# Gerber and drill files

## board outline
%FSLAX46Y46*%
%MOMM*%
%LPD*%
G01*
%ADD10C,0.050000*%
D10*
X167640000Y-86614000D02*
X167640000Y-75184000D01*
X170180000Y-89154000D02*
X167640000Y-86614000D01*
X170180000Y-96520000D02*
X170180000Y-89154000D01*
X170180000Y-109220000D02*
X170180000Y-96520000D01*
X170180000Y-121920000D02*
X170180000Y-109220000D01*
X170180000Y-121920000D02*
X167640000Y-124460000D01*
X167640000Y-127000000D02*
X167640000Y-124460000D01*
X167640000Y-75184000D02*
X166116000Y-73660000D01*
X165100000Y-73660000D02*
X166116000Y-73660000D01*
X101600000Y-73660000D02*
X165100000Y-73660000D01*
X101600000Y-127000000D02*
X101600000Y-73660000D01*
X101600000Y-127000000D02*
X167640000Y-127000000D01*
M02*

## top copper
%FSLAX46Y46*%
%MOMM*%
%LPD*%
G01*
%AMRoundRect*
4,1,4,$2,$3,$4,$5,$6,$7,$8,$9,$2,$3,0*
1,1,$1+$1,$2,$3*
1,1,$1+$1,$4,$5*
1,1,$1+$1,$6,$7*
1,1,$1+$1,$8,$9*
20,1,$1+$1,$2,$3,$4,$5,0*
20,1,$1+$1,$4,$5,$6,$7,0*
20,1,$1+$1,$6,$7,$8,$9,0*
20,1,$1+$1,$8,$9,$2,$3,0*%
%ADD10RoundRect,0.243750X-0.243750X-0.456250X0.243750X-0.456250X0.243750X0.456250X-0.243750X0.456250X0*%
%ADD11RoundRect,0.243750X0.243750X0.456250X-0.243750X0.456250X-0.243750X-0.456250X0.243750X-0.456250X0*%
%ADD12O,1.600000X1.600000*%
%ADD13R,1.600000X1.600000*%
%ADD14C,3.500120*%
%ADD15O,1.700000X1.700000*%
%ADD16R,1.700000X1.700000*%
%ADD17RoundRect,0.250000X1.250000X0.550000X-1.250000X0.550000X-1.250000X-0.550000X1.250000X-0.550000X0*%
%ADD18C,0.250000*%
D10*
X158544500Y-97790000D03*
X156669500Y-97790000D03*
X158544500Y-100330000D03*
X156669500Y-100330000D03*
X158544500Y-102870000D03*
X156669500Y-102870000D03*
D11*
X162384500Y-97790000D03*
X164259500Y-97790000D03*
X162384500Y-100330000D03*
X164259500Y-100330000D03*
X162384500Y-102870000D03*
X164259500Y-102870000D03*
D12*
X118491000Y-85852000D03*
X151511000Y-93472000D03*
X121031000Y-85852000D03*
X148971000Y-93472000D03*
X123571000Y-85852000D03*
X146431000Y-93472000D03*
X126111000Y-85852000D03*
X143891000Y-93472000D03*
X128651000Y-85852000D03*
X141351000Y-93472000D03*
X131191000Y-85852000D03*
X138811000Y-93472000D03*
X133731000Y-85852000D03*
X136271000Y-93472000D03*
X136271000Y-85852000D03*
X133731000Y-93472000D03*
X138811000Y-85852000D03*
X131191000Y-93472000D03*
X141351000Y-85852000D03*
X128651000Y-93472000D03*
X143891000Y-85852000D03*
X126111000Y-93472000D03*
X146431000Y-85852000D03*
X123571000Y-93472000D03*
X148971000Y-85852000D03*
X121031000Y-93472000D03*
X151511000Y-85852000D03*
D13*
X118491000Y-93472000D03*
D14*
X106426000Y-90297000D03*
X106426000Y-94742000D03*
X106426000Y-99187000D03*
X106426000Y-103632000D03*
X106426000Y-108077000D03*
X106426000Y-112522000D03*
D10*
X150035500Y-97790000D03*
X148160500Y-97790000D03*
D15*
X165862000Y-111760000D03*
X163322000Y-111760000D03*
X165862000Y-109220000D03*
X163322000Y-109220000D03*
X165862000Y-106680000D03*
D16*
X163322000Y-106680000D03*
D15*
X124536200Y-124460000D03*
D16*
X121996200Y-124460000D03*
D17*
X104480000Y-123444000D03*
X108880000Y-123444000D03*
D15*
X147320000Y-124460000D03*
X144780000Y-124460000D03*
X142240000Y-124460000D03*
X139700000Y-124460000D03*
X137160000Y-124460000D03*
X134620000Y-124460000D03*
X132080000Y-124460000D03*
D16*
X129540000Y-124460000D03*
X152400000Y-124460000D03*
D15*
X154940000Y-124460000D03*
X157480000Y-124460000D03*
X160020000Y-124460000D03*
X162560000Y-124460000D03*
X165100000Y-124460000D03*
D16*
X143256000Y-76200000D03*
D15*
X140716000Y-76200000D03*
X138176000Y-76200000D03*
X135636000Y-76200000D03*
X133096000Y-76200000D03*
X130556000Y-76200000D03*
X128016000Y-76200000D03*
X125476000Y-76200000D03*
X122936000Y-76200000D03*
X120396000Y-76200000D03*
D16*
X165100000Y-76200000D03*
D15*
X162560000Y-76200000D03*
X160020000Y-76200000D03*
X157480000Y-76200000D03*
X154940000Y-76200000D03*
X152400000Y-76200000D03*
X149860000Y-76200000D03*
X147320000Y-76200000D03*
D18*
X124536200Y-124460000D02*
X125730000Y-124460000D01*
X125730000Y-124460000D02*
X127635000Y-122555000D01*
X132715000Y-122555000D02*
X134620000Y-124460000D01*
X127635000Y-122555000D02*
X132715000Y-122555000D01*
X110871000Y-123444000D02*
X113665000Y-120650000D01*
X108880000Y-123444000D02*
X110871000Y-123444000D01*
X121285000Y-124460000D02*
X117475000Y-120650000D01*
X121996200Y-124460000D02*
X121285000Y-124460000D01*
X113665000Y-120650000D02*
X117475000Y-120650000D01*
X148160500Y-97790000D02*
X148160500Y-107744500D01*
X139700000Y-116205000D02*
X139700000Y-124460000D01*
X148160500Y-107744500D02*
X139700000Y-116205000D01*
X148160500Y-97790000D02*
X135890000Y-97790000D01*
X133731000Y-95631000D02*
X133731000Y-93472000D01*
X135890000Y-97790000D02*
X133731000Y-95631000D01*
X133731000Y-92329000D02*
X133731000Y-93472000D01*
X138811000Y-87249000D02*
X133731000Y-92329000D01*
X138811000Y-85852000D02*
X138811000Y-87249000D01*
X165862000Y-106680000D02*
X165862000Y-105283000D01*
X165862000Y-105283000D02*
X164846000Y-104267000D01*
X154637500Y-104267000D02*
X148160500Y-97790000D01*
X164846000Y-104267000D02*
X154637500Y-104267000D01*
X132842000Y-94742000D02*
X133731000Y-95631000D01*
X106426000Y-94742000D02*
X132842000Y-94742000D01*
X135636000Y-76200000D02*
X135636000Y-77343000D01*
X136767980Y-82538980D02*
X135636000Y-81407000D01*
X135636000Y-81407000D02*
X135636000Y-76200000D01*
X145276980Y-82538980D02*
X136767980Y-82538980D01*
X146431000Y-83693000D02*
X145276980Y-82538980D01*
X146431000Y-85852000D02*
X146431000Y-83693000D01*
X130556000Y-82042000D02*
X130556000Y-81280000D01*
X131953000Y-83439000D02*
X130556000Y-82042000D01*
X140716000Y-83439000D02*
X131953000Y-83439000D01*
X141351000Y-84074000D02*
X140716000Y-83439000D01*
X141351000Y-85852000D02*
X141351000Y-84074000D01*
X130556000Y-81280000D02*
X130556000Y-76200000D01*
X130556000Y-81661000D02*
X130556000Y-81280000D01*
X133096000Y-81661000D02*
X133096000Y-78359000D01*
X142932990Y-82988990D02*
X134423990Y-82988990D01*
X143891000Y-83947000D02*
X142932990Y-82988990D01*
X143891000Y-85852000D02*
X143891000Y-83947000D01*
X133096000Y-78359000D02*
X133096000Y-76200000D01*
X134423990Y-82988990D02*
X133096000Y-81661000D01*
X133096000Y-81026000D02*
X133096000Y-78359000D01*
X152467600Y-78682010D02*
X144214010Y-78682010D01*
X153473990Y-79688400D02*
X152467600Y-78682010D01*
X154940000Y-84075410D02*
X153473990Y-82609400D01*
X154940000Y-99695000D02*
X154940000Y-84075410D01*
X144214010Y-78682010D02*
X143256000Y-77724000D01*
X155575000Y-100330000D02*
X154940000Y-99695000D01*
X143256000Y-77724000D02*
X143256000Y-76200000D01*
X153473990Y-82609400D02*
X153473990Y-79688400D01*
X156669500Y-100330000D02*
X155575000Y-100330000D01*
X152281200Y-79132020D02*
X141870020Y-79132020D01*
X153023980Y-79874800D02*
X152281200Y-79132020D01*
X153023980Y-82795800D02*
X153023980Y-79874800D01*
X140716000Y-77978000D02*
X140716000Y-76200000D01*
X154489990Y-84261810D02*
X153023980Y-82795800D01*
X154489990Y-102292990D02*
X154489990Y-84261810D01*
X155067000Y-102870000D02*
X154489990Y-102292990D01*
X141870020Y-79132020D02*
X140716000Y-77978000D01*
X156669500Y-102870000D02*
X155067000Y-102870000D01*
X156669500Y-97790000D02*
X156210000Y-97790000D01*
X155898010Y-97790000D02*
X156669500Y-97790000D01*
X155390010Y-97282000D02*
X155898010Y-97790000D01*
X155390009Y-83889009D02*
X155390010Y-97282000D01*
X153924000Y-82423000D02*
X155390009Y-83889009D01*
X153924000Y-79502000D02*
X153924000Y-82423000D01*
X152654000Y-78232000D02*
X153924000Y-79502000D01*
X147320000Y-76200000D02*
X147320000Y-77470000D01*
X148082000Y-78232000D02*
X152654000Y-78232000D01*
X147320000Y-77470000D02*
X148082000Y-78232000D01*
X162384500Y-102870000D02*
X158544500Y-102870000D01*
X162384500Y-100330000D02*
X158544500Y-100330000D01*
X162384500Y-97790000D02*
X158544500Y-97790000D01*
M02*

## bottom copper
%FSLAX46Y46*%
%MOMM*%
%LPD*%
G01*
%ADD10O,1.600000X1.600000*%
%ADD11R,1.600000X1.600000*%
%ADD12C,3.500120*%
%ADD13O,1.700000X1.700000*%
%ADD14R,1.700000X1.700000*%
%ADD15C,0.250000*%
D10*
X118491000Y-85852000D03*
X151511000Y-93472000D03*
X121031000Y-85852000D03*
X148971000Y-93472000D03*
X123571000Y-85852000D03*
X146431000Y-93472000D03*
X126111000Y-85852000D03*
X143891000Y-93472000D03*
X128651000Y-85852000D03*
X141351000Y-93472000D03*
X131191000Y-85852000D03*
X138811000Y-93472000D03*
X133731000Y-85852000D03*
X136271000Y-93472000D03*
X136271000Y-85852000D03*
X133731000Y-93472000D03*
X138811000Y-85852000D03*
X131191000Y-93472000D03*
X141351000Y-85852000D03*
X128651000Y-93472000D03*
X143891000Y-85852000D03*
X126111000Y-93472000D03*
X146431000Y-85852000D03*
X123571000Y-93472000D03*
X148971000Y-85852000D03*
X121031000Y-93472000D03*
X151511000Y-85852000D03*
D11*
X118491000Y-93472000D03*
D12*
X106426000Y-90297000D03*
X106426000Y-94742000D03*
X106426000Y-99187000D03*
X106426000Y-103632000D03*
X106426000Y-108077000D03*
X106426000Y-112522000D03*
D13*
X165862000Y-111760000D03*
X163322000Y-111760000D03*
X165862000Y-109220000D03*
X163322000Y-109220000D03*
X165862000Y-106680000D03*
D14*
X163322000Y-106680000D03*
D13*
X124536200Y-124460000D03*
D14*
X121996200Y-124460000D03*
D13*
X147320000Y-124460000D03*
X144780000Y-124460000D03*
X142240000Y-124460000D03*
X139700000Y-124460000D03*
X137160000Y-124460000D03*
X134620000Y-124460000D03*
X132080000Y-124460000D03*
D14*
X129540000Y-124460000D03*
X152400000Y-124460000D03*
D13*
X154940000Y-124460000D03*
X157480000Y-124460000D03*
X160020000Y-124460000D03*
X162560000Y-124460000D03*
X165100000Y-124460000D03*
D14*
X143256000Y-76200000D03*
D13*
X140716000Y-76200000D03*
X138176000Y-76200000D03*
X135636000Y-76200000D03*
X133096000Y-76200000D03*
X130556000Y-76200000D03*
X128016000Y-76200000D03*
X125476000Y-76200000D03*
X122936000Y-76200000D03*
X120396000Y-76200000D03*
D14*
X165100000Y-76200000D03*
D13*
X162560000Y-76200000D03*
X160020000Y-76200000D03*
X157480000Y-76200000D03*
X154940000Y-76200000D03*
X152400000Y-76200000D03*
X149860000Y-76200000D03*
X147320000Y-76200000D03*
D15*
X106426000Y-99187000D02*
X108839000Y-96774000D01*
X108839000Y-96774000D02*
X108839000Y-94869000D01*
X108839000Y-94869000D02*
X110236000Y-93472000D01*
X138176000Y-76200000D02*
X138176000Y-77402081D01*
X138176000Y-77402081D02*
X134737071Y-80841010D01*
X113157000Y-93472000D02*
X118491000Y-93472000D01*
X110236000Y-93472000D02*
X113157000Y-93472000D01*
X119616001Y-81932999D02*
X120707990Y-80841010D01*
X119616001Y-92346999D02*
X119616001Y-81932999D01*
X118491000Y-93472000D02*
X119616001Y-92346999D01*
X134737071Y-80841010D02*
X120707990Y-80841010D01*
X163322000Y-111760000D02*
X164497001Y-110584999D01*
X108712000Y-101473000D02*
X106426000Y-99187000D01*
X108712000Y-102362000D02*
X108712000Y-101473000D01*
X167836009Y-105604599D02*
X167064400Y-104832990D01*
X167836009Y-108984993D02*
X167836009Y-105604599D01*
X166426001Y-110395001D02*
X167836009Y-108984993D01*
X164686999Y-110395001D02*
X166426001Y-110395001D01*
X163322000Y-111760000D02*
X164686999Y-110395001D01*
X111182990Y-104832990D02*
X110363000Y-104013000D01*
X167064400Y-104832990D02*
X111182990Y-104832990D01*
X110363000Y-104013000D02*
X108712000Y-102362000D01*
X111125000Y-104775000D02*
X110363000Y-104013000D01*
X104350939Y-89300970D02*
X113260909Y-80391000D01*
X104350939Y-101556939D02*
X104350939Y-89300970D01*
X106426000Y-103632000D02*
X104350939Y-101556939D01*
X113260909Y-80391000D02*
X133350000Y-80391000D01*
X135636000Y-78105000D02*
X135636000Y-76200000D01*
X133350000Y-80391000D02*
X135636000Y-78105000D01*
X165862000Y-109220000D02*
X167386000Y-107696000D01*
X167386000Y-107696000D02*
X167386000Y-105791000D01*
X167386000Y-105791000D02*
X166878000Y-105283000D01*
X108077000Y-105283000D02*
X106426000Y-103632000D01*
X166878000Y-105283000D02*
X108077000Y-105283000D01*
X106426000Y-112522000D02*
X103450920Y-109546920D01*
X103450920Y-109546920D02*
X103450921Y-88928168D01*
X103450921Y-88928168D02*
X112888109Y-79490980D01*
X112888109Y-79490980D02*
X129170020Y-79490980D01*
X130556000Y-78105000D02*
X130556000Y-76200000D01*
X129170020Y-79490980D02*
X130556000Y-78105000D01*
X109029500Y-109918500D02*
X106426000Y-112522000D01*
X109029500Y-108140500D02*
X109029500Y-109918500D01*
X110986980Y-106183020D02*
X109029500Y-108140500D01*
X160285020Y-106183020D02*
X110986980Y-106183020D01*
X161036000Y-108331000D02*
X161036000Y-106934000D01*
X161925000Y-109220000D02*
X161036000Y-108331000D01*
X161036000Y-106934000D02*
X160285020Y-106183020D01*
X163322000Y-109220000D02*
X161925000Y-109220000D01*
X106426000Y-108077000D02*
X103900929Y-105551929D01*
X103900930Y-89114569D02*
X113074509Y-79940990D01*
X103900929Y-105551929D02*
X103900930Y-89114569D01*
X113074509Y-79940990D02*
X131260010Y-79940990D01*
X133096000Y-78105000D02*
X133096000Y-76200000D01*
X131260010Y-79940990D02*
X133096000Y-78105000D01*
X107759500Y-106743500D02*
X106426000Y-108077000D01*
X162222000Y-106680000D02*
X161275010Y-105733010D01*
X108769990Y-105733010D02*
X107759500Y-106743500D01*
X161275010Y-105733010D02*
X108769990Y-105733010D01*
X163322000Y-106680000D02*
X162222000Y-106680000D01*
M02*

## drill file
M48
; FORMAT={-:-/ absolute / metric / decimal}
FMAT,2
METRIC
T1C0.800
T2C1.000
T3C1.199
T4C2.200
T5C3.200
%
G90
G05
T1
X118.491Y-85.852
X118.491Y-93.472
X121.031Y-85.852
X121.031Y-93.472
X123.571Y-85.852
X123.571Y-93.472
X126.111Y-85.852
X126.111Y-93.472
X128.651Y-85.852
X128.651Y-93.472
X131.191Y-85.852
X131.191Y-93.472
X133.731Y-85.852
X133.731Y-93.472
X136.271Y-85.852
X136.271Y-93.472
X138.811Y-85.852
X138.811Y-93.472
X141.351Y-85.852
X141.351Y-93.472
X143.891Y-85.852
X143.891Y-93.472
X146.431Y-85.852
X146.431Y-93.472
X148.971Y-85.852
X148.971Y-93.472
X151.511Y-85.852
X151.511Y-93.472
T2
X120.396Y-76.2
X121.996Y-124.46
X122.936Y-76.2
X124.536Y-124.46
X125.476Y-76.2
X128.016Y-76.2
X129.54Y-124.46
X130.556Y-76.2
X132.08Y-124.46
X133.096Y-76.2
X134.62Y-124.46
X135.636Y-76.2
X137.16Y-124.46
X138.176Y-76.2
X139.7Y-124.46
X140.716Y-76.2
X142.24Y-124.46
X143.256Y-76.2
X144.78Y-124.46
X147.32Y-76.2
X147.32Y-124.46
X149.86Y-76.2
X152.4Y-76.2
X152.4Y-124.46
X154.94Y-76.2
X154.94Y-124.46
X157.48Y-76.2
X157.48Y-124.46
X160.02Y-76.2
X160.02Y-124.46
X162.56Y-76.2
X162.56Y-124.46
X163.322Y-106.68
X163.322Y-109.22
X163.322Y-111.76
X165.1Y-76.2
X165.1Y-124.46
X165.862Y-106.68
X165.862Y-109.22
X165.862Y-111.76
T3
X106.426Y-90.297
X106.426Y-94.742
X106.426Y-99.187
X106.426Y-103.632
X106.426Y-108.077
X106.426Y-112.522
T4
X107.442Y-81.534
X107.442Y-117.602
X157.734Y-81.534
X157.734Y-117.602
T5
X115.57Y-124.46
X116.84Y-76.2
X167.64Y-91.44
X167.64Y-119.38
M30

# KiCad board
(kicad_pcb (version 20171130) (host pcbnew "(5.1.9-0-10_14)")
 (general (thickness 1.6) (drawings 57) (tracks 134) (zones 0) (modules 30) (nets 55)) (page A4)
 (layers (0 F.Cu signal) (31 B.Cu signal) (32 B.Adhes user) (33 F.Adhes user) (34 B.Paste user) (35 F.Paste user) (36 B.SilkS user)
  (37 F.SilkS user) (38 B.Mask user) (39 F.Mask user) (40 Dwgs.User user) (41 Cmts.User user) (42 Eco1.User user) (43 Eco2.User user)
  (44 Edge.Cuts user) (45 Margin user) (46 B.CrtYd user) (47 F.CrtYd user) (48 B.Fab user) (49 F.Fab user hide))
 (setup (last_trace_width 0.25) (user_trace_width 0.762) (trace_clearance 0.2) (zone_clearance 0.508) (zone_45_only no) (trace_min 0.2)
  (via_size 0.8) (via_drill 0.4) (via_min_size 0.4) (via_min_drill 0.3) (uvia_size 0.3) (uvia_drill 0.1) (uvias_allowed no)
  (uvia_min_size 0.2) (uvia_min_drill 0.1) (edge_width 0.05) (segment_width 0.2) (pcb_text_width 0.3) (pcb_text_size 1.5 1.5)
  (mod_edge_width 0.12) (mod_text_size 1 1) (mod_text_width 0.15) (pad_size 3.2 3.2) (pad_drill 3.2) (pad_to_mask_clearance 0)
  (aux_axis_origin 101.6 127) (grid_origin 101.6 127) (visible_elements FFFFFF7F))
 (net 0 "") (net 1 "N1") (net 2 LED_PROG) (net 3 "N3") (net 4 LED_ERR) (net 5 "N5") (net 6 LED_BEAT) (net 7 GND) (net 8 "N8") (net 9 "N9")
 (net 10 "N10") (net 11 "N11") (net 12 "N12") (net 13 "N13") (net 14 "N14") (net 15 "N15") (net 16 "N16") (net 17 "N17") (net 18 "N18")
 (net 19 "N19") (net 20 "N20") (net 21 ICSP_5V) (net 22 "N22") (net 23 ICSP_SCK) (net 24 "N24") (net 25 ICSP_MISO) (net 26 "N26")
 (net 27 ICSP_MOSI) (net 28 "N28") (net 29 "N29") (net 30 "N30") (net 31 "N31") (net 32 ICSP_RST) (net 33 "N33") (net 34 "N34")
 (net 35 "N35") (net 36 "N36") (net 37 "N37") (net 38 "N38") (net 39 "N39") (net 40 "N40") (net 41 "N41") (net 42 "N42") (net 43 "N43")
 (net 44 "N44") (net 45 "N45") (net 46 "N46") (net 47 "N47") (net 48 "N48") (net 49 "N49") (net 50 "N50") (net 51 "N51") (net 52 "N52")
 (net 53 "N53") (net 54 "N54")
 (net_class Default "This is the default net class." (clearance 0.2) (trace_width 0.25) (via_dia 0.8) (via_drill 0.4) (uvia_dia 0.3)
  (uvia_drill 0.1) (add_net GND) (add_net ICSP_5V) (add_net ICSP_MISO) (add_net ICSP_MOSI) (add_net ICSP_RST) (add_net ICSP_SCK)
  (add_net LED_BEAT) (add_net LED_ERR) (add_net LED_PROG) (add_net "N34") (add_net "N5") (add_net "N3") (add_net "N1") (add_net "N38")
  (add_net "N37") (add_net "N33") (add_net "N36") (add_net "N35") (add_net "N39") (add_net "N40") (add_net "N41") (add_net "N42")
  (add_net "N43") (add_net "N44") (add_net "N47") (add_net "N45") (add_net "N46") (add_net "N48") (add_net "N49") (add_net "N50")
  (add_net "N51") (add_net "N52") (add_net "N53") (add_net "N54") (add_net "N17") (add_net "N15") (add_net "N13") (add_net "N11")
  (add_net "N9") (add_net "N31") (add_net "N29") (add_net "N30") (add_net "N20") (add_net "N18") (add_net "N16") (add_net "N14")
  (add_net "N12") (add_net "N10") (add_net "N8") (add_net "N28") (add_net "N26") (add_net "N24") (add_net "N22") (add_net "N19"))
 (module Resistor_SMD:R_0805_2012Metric (layer F.Cu) (at 157.607 97.79)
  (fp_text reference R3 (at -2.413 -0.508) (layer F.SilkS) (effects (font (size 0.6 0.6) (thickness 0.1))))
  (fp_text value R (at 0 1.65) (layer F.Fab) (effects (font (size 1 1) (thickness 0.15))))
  (pad 2 smd roundrect (at 0.9375 0) (size 0.975 1.4) (layers F.Cu F.Paste F.Mask) (roundrect_rratio 0.25) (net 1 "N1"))
  (pad 1 smd roundrect (at -0.9375 0) (size 0.975 1.4) (layers F.Cu F.Paste F.Mask) (roundrect_rratio 0.25) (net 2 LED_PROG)))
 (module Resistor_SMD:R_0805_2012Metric (layer F.Cu) (at 157.607 100.33)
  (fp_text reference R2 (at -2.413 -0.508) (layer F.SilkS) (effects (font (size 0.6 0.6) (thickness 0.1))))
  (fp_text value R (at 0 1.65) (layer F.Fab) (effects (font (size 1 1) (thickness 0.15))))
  (pad 2 smd roundrect (at 0.9375 0) (size 0.975 1.4) (layers F.Cu F.Paste F.Mask) (roundrect_rratio 0.25) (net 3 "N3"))
  (pad 1 smd roundrect (at -0.9375 0) (size 0.975 1.4) (layers F.Cu F.Paste F.Mask) (roundrect_rratio 0.25) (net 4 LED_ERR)))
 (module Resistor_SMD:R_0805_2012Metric (layer F.Cu) (at 157.607 102.87)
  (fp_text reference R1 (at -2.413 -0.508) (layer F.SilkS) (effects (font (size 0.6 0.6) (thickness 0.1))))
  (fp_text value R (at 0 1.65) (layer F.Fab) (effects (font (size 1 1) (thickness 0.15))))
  (pad 2 smd roundrect (at 0.9375 0) (size 0.975 1.4) (layers F.Cu F.Paste F.Mask) (roundrect_rratio 0.25) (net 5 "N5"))
  (pad 1 smd roundrect (at -0.9375 0) (size 0.975 1.4) (layers F.Cu F.Paste F.Mask) (roundrect_rratio 0.25) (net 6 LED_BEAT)))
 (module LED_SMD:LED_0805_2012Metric (layer F.Cu) (at 163.322 97.79 180)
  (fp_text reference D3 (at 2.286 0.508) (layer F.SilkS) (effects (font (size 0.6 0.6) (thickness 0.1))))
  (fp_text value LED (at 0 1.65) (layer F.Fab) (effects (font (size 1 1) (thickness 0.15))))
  (pad 2 smd roundrect (at 0.9375 0 180) (size 0.975 1.4) (layers F.Cu F.Paste F.Mask) (roundrect_rratio 0.25) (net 1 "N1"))
  (pad 1 smd roundrect (at -0.9375 0 180) (size 0.975 1.4) (layers F.Cu F.Paste F.Mask) (roundrect_rratio 0.25) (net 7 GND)))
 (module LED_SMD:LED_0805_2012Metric (layer F.Cu) (at 163.322 100.33 180)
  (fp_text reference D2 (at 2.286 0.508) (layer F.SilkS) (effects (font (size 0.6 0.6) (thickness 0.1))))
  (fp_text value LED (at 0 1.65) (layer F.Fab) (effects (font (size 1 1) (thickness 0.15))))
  (pad 2 smd roundrect (at 0.9375 0 180) (size 0.975 1.4) (layers F.Cu F.Paste F.Mask) (roundrect_rratio 0.25) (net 3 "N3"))
  (pad 1 smd roundrect (at -0.9375 0 180) (size 0.975 1.4) (layers F.Cu F.Paste F.Mask) (roundrect_rratio 0.25) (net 7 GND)))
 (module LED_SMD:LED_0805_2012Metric (layer F.Cu) (at 163.322 102.87 180)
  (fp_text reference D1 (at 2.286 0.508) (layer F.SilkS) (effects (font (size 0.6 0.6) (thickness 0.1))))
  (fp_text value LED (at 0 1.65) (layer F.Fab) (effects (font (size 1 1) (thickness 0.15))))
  (pad 2 smd roundrect (at 0.9375 0 180) (size 0.975 1.4) (layers F.Cu F.Paste F.Mask) (roundrect_rratio 0.25) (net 5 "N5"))
  (pad 1 smd roundrect (at -0.9375 0 180) (size 0.975 1.4) (layers F.Cu F.Paste F.Mask) (roundrect_rratio 0.25) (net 7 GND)))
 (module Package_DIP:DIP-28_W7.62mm (layer F.Cu) (at 118.491 93.472 90)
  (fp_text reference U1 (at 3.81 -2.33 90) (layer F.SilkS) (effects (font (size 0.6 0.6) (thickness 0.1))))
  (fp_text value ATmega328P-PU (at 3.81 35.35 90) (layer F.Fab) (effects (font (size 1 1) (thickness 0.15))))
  (pad 28 thru_hole oval (at 7.62 0 90) (size 1.6 1.6) (drill 0.8) (layers *.Cu *.Mask) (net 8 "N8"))
  (pad 14 thru_hole oval (at 0 33.02 90) (size 1.6 1.6) (drill 0.8) (layers *.Cu *.Mask) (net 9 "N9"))
  (pad 27 thru_hole oval (at 7.62 2.54 90) (size 1.6 1.6) (drill 0.8) (layers *.Cu *.Mask) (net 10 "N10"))
  (pad 13 thru_hole oval (at 0 30.48 90) (size 1.6 1.6) (drill 0.8) (layers *.Cu *.Mask) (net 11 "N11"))
  (pad 26 thru_hole oval (at 7.62 5.08 90) (size 1.6 1.6) (drill 0.8) (layers *.Cu *.Mask) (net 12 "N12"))
  (pad 12 thru_hole oval (at 0 27.94 90) (size 1.6 1.6) (drill 0.8) (layers *.Cu *.Mask) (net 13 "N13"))
  (pad 25 thru_hole oval (at 7.62 7.62 90) (size 1.6 1.6) (drill 0.8) (layers *.Cu *.Mask) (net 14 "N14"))
  (pad 11 thru_hole oval (at 0 25.4 90) (size 1.6 1.6) (drill 0.8) (layers *.Cu *.Mask) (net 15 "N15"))
  (pad 24 thru_hole oval (at 7.62 10.16 90) (size 1.6 1.6) (drill 0.8) (layers *.Cu *.Mask) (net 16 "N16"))
  (pad 10 thru_hole oval (at 0 22.86 90) (size 1.6 1.6) (drill 0.8) (layers *.Cu *.Mask) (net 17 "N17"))
  (pad 23 thru_hole oval (at 7.62 12.7 90) (size 1.6 1.6) (drill 0.8) (layers *.Cu *.Mask) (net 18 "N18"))
  (pad 9 thru_hole oval (at 0 20.32 90) (size 1.6 1.6) (drill 0.8) (layers *.Cu *.Mask) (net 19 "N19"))
  (pad 22 thru_hole oval (at 7.62 15.24 90) (size 1.6 1.6) (drill 0.8) (layers *.Cu *.Mask) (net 7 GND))
  (pad 8 thru_hole oval (at 0 17.78 90) (size 1.6 1.6) (drill 0.8) (layers *.Cu *.Mask) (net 7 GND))
  (pad 21 thru_hole oval (at 7.62 17.78 90) (size 1.6 1.6) (drill 0.8) (layers *.Cu *.Mask) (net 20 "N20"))
  (pad 7 thru_hole oval (at 0 15.24 90) (size 1.6 1.6) (drill 0.8) (layers *.Cu *.Mask) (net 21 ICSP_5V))
  (pad 20 thru_hole oval (at 7.62 20.32 90) (size 1.6 1.6) (drill 0.8) (layers *.Cu *.Mask) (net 21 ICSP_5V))
  (pad 6 thru_hole oval (at 0 12.7 90) (size 1.6 1.6) (drill 0.8) (layers *.Cu *.Mask) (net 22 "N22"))
  (pad 19 thru_hole oval (at 7.62 22.86 90) (size 1.6 1.6) (drill 0.8) (layers *.Cu *.Mask) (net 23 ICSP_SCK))
  (pad 5 thru_hole oval (at 0 10.16 90) (size 1.6 1.6) (drill 0.8) (layers *.Cu *.Mask) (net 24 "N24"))
  (pad 18 thru_hole oval (at 7.62 25.4 90) (size 1.6 1.6) (drill 0.8) (layers *.Cu *.Mask) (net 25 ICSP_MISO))
  (pad 4 thru_hole oval (at 0 7.62 90) (size 1.6 1.6) (drill 0.8) (layers *.Cu *.Mask) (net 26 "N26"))
  (pad 17 thru_hole oval (at 7.62 27.94 90) (size 1.6 1.6) (drill 0.8) (layers *.Cu *.Mask) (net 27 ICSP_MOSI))
  (pad 3 thru_hole oval (at 0 5.08 90) (size 1.6 1.6) (drill 0.8) (layers *.Cu *.Mask) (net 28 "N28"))
  (pad 16 thru_hole oval (at 7.62 30.48 90) (size 1.6 1.6) (drill 0.8) (layers *.Cu *.Mask) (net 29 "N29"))
  (pad 2 thru_hole oval (at 0 2.54 90) (size 1.6 1.6) (drill 0.8) (layers *.Cu *.Mask) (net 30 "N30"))
  (pad 15 thru_hole oval (at 7.62 33.02 90) (size 1.6 1.6) (drill 0.8) (layers *.Cu *.Mask) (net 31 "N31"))
  (pad 1 thru_hole rect (at 0 0 90) (size 1.6 1.6) (drill 0.8) (layers *.Cu *.Mask) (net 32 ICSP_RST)))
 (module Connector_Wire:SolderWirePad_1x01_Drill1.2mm (layer F.Cu) (at 106.426 90.297 90)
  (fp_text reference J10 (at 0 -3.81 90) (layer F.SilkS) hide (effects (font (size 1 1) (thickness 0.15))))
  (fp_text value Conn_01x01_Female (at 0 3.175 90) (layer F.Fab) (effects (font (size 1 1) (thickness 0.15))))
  (pad 1 thru_hole circle (at 0 0 90) (size 3.50012 3.50012) (drill 1.19888) (layers *.Cu *.Mask) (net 7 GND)))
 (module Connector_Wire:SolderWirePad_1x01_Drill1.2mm (layer F.Cu) (at 106.426 94.742 90)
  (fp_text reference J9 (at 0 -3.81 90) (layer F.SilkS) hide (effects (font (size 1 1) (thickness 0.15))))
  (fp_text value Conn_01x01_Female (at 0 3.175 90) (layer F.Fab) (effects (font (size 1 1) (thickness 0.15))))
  (pad 1 thru_hole circle (at 0 0 90) (size 3.50012 3.50012) (drill 1.19888) (layers *.Cu *.Mask) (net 21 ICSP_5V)))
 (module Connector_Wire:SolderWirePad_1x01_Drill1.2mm (layer F.Cu) (at 106.426 99.187 90)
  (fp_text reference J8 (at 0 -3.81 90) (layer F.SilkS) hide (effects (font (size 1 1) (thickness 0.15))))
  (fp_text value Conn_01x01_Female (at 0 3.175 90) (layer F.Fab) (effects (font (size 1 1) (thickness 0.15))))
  (pad 1 thru_hole circle (at 0 0 90) (size 3.50012 3.50012) (drill 1.19888) (layers *.Cu *.Mask) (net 32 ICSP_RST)))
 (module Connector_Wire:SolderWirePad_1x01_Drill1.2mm (layer F.Cu) (at 106.426 103.632 90)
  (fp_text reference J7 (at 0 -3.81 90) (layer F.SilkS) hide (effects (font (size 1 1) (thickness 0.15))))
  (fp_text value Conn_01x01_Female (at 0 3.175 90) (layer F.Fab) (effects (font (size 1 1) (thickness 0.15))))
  (pad 1 thru_hole circle (at 0 0 90) (size 3.50012 3.50012) (drill 1.19888) (layers *.Cu *.Mask) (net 27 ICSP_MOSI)))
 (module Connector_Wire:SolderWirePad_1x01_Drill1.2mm (layer F.Cu) (at 106.426 108.077 90)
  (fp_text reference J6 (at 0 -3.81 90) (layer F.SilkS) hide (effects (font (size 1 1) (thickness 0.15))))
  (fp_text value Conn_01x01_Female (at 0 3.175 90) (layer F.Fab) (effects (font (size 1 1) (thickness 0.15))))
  (pad 1 thru_hole circle (at 0 0 90) (size 3.50012 3.50012) (drill 1.19888) (layers *.Cu *.Mask) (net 25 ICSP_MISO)))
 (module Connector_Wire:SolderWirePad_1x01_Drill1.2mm (layer F.Cu) (at 106.426 112.522 90)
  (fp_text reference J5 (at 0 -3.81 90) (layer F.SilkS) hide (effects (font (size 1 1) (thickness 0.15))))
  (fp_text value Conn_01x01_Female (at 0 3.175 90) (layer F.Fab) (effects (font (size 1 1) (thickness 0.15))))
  (pad 1 thru_hole circle (at 0 0 90) (size 3.50012 3.50012) (drill 1.19888) (layers *.Cu *.Mask) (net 23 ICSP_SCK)))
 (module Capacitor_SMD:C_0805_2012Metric (layer F.Cu) (at 149.098 97.79)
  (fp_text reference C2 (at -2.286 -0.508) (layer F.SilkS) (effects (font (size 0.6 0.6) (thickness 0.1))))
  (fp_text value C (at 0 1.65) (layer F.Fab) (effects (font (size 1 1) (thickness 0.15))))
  (pad 2 smd roundrect (at 0.9375 0) (size 0.975 1.4) (layers F.Cu F.Paste F.Mask) (roundrect_rratio 0.25) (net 7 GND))
  (pad 1 smd roundrect (at -0.9375 0) (size 0.975 1.4) (layers F.Cu F.Paste F.Mask) (roundrect_rratio 0.25) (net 21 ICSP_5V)))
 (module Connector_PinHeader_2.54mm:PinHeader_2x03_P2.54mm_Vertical (layer F.Cu) (at 163.322 106.68)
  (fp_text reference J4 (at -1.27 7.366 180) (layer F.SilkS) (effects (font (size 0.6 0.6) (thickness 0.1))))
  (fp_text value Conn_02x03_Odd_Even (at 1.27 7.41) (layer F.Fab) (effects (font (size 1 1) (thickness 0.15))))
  (pad 6 thru_hole oval (at 2.54 5.08) (size 1.7 1.7) (drill 1) (layers *.Cu *.Mask) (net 7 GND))
  (pad 5 thru_hole oval (at 0 5.08) (size 1.7 1.7) (drill 1) (layers *.Cu *.Mask) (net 32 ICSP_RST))
  (pad 4 thru_hole oval (at 2.54 2.54) (size 1.7 1.7) (drill 1) (layers *.Cu *.Mask) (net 27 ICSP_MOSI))
  (pad 3 thru_hole oval (at 0 2.54) (size 1.7 1.7) (drill 1) (layers *.Cu *.Mask) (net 23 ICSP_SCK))
  (pad 2 thru_hole oval (at 2.54 0) (size 1.7 1.7) (drill 1) (layers *.Cu *.Mask) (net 21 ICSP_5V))
  (pad 1 thru_hole rect (at 0 0) (size 1.7 1.7) (drill 1) (layers *.Cu *.Mask) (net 25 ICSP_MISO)))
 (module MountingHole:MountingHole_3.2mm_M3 (layer F.Cu) (at 115.57 124.46)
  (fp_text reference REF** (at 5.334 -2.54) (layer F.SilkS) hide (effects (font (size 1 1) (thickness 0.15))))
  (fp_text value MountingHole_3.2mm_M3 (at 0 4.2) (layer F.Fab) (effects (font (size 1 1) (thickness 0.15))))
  (pad 1 np_thru_hole circle (at 0 0) (size 3.2 3.2) (drill 3.2) (layers *.Cu *.Mask)))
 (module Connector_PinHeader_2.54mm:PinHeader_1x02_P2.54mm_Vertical (layer F.Cu) (at 121.9962 124.46 90)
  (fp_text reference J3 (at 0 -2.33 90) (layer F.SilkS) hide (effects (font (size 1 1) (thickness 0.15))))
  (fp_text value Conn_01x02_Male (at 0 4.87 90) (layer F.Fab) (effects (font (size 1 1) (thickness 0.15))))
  (pad 2 thru_hole oval (at 0 2.54 90) (size 1.7 1.7) (drill 1) (layers *.Cu *.Mask) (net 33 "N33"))
  (pad 1 thru_hole rect (at 0 0 90) (size 1.7 1.7) (drill 1) (layers *.Cu *.Mask) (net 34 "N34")))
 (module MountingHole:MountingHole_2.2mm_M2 (layer F.Cu) (at 107.442 117.602)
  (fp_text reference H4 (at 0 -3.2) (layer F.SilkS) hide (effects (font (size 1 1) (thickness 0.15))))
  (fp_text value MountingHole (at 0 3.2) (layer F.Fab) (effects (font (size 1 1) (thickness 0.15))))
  (pad 1 np_thru_hole circle (at 0 0) (size 2.2 2.2) (drill 2.2) (layers *.Cu *.Mask)))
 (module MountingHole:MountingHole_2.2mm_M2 (layer F.Cu) (at 107.442 81.534)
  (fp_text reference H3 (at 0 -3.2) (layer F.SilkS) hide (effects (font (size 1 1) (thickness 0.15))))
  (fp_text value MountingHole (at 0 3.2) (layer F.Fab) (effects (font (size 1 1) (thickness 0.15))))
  (pad 1 np_thru_hole circle (at 0 0) (size 2.2 2.2) (drill 2.2) (layers *.Cu *.Mask)))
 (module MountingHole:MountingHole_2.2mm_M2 (layer F.Cu) (at 157.734 81.534)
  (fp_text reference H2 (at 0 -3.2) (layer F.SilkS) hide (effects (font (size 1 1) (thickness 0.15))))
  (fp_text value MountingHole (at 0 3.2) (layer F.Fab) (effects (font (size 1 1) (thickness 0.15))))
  (pad 1 np_thru_hole circle (at 0 0) (size 2.2 2.2) (drill 2.2) (layers *.Cu *.Mask)))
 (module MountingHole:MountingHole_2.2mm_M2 (layer F.Cu) (at 157.734 117.602)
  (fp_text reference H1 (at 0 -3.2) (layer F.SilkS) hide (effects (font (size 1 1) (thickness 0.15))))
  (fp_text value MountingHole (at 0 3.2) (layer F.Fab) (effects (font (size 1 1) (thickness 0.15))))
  (pad 1 np_thru_hole circle (at 0 0) (size 2.2 2.2) (drill 2.2) (layers *.Cu *.Mask)))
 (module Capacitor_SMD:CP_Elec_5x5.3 (layer F.Cu) (at 106.68 123.444 180)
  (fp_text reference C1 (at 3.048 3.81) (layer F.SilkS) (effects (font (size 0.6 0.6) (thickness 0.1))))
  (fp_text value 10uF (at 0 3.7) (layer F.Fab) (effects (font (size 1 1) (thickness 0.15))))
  (pad 2 smd roundrect (at 2.2 0 180) (size 3 1.6) (layers F.Cu F.Paste F.Mask) (roundrect_rratio 0.15625) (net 7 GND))
  (pad 1 smd roundrect (at -2.2 0 180) (size 3 1.6) (layers F.Cu F.Paste F.Mask) (roundrect_rratio 0.15625) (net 34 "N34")))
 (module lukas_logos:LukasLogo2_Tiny (layer F.Cu) (at 157.988 109.22 90)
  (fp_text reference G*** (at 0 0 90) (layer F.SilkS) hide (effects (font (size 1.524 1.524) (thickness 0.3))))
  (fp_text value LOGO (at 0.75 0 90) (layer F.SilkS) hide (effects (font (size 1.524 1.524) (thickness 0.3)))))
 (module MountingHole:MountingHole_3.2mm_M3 (layer F.Cu) (at 116.84 76.2)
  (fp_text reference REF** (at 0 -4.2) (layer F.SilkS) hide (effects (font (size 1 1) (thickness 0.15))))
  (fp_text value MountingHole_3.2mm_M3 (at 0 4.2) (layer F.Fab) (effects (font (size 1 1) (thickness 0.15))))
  (pad 1 np_thru_hole circle (at 0 0) (size 3.2 3.2) (drill 3.2) (layers *.Cu *.Mask)))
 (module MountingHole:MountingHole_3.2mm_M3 (layer F.Cu) (at 167.64 91.44)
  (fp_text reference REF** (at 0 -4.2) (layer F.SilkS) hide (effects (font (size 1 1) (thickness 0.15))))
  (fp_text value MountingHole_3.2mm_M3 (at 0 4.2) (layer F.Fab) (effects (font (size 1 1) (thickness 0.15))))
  (pad 1 np_thru_hole circle (at 0 0) (size 3.2 3.2) (drill 3.2) (layers *.Cu *.Mask)))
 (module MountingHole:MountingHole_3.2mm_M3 (layer F.Cu) (at 167.64 119.38)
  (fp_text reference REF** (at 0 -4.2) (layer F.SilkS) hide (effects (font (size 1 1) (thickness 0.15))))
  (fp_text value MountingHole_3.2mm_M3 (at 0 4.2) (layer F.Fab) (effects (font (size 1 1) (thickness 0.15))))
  (pad 1 np_thru_hole circle (at 0 0) (size 3.2 3.2) (drill 3.2) (layers *.Cu *.Mask)))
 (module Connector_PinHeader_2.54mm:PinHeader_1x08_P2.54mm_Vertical (layer F.Cu) (at 129.54 124.46 90)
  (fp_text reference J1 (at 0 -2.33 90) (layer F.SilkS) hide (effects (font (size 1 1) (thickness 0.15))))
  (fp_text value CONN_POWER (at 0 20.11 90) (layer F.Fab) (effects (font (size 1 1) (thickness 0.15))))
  (pad 8 thru_hole oval (at 0 17.78 90) (size 1.7 1.7) (drill 1) (layers *.Cu *.Mask) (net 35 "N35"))
  (pad 7 thru_hole oval (at 0 15.24 90) (size 1.7 1.7) (drill 1) (layers *.Cu *.Mask) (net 7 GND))
  (pad 6 thru_hole oval (at 0 12.7 90) (size 1.7 1.7) (drill 1) (layers *.Cu *.Mask) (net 7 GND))
  (pad 5 thru_hole oval (at 0 10.16 90) (size 1.7 1.7) (drill 1) (layers *.Cu *.Mask) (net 21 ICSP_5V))
  (pad 4 thru_hole oval (at 0 7.62 90) (size 1.7 1.7) (drill 1) (layers *.Cu *.Mask) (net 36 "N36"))
  (pad 3 thru_hole oval (at 0 5.08 90) (size 1.7 1.7) (drill 1) (layers *.Cu *.Mask) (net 33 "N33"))
  (pad 2 thru_hole oval (at 0 2.54 90) (size 1.7 1.7) (drill 1) (layers *.Cu *.Mask) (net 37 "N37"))
  (pad 1 thru_hole rect (at 0 0 90) (size 1.7 1.7) (drill 1) (layers *.Cu *.Mask) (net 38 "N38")))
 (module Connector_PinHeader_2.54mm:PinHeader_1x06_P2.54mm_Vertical (layer F.Cu) (at 152.4 124.46 90)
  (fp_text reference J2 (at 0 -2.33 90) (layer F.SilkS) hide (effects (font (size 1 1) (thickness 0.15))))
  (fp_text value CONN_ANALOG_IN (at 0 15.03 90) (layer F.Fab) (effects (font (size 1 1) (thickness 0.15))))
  (pad 1 thru_hole rect (at 0 0 90) (size 1.7 1.7) (drill 1) (layers *.Cu *.Mask) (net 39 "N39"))
  (pad 2 thru_hole oval (at 0 2.54 90) (size 1.7 1.7) (drill 1) (layers *.Cu *.Mask) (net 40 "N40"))
  (pad 3 thru_hole oval (at 0 5.08 90) (size 1.7 1.7) (drill 1) (layers *.Cu *.Mask) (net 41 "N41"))
  (pad 4 thru_hole oval (at 0 7.62 90) (size 1.7 1.7) (drill 1) (layers *.Cu *.Mask) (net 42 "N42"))
  (pad 5 thru_hole oval (at 0 10.16 90) (size 1.7 1.7) (drill 1) (layers *.Cu *.Mask) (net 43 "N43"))
  (pad 6 thru_hole oval (at 0 12.7 90) (size 1.7 1.7) (drill 1) (layers *.Cu *.Mask) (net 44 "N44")))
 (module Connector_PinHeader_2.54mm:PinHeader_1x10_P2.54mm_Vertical (layer F.Cu) (at 143.256 76.2 270)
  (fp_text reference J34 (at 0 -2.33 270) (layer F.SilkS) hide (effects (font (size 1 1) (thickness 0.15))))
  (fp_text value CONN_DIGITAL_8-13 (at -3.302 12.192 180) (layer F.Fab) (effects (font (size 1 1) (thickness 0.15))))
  (pad 1 thru_hole rect (at 0 0 270) (size 1.7 1.7) (drill 1) (layers *.Cu *.Mask) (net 4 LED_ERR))
  (pad 2 thru_hole oval (at 0 2.54 270) (size 1.7 1.7) (drill 1) (layers *.Cu *.Mask) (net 6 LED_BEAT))
  (pad 3 thru_hole oval (at 0 5.08 270) (size 1.7 1.7) (drill 1) (layers *.Cu *.Mask) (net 32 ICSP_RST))
  (pad 4 thru_hole oval (at 0 7.62 270) (size 1.7 1.7) (drill 1) (layers *.Cu *.Mask) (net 27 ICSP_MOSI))
  (pad 5 thru_hole oval (at 0 10.16 270) (size 1.7 1.7) (drill 1) (layers *.Cu *.Mask) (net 25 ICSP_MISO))
  (pad 6 thru_hole oval (at 0 12.7 270) (size 1.7 1.7) (drill 1) (layers *.Cu *.Mask) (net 23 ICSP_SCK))
  (pad 7 thru_hole oval (at 0 15.24 270) (size 1.7 1.7) (drill 1) (layers *.Cu *.Mask) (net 7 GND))
  (pad 8 thru_hole oval (at 0 17.78 270) (size 1.7 1.7) (drill 1) (layers *.Cu *.Mask) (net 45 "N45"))
  (pad 9 thru_hole oval (at 0 20.32 270) (size 1.7 1.7) (drill 1) (layers *.Cu *.Mask) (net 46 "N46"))
  (pad 10 thru_hole oval (at 0 22.86 270) (size 1.7 1.7) (drill 1) (layers *.Cu *.Mask) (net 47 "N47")))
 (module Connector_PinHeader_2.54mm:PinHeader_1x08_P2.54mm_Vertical (layer F.Cu) (at 165.1 76.2 270)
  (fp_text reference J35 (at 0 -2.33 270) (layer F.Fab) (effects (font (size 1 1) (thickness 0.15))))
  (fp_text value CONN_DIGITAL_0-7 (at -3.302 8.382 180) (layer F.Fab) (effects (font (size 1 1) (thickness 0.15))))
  (pad 1 thru_hole rect (at 0 0 270) (size 1.7 1.7) (drill 1) (layers *.Cu *.Mask) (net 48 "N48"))
  (pad 2 thru_hole oval (at 0 2.54 270) (size 1.7 1.7) (drill 1) (layers *.Cu *.Mask) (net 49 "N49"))
  (pad 3 thru_hole oval (at 0 5.08 270) (size 1.7 1.7) (drill 1) (layers *.Cu *.Mask) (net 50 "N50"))
  (pad 4 thru_hole oval (at 0 7.62 270) (size 1.7 1.7) (drill 1) (layers *.Cu *.Mask) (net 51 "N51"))
  (pad 5 thru_hole oval (at 0 10.16 270) (size 1.7 1.7) (drill 1) (layers *.Cu *.Mask) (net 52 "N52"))
  (pad 6 thru_hole oval (at 0 12.7 270) (size 1.7 1.7) (drill 1) (layers *.Cu *.Mask) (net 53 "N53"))
  (pad 7 thru_hole oval (at 0 15.24 270) (size 1.7 1.7) (drill 1) (layers *.Cu *.Mask) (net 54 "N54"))
  (pad 8 thru_hole oval (at 0 17.78 270) (size 1.7 1.7) (drill 1) (layers *.Cu *.Mask) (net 2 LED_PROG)))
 (gr_line (start 167.64 86.614) (end 167.64 75.184) (layer Edge.Cuts) (width 0.05))
 (gr_line (start 170.18 89.154) (end 167.64 86.614) (layer Edge.Cuts) (width 0.05))
 (gr_line (start 170.18 96.52) (end 170.18 89.154) (layer Edge.Cuts) (width 0.05))
 (gr_line (start 170.18 109.22) (end 170.18 96.52) (layer Edge.Cuts) (width 0.05))
 (gr_line (start 170.18 121.92) (end 170.18 109.22) (layer Edge.Cuts) (width 0.05))
 (gr_line (start 170.18 121.92) (end 167.64 124.46) (layer Edge.Cuts) (width 0.05))
 (gr_line (start 167.64 127) (end 167.64 124.46) (layer Edge.Cuts) (width 0.05))
 (gr_line (start 167.64 75.184) (end 166.116 73.66) (layer Edge.Cuts) (width 0.05))
 (gr_line (start 165.1 73.66) (end 166.116 73.66) (layer Edge.Cuts) (width 0.05))
 (gr_line (start 101.6 73.66) (end 165.1 73.66) (layer Edge.Cuts) (width 0.05))
 (gr_line (start 101.6 127) (end 101.6 73.66) (layer Edge.Cuts) (width 0.05))
 (gr_line (start 101.6 127) (end 167.64 127) (layer Edge.Cuts) (width 0.05))
 (segment (start 124.5362 124.46) (end 125.73 124.46) (width 0.25) (layer F.Cu) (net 33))
 (segment (start 125.73 124.46) (end 127.635 122.555) (width 0.25) (layer F.Cu) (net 33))
 (segment (start 132.715 122.555) (end 134.62 124.46) (width 0.25) (layer F.Cu) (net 33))
 (segment (start 127.635 122.555) (end 132.715 122.555) (width 0.25) (layer F.Cu) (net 33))
 (segment (start 110.871 123.444) (end 113.665 120.65) (width 0.25) (layer F.Cu) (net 34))
 (segment (start 108.88 123.444) (end 110.871 123.444) (width 0.25) (layer F.Cu) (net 34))
 (segment (start 121.285 124.46) (end 117.475 120.65) (width 0.25) (layer F.Cu) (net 34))
 (segment (start 121.9962 124.46) (end 121.285 124.46) (width 0.25) (layer F.Cu) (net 34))
 (segment (start 113.665 120.65) (end 117.475 120.65) (width 0.25) (layer F.Cu) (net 34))
 (segment (start 148.1605 97.79) (end 148.1605 107.7445) (width 0.25) (layer F.Cu) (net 21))
 (segment (start 139.7 116.205) (end 139.7 124.46) (width 0.25) (layer F.Cu) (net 21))
 (segment (start 148.1605 107.7445) (end 139.7 116.205) (width 0.25) (layer F.Cu) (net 21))
 (segment (start 148.1605 97.79) (end 135.89 97.79) (width 0.25) (layer F.Cu) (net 21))
 (segment (start 133.731 95.631) (end 133.731 93.472) (width 0.25) (layer F.Cu) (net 21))
 (segment (start 135.89 97.79) (end 133.731 95.631) (width 0.25) (layer F.Cu) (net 21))
 (segment (start 133.731 92.329) (end 133.731 93.472) (width 0.25) (layer F.Cu) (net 21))
 (segment (start 138.811 87.249) (end 133.731 92.329) (width 0.25) (layer F.Cu) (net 21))
 (segment (start 138.811 85.852) (end 138.811 87.249) (width 0.25) (layer F.Cu) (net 21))
 (segment (start 165.862 106.68) (end 165.862 105.283) (width 0.25) (layer F.Cu) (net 21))
 (segment (start 165.862 105.283) (end 164.846 104.267) (width 0.25) (layer F.Cu) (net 21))
 (segment (start 154.6375 104.267) (end 148.1605 97.79) (width 0.25) (layer F.Cu) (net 21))
 (segment (start 164.846 104.267) (end 154.6375 104.267) (width 0.25) (layer F.Cu) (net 21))
 (segment (start 132.842 94.742) (end 133.731 95.631) (width 0.25) (layer F.Cu) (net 21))
 (segment (start 106.426 94.742) (end 132.842 94.742) (width 0.25) (layer F.Cu) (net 21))
 (segment (start 106.426 99.187) (end 108.839 96.774) (width 0.25) (layer B.Cu) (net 32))
 (segment (start 108.839 96.774) (end 108.839 94.869) (width 0.25) (layer B.Cu) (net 32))
 (segment (start 108.839 94.869) (end 110.236 93.472) (width 0.25) (layer B.Cu) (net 32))
 (segment (start 138.176 76.2) (end 138.176 77.402081) (width 0.25) (layer B.Cu) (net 32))
 (segment (start 138.176 77.402081) (end 134.737071 80.84101) (width 0.25) (layer B.Cu) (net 32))
 (segment (start 113.157 93.472) (end 118.491 93.472) (width 0.25) (layer B.Cu) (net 32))
 (segment (start 110.236 93.472) (end 113.157 93.472) (width 0.25) (layer B.Cu) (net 32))
 (segment (start 119.616001 81.932999) (end 120.70799 80.84101) (width 0.25) (layer B.Cu) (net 32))
 (segment (start 119.616001 92.346999) (end 119.616001 81.932999) (width 0.25) (layer B.Cu) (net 32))
 (segment (start 118.491 93.472) (end 119.616001 92.346999) (width 0.25) (layer B.Cu) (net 32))
 (segment (start 134.737071 80.84101) (end 120.70799 80.84101) (width 0.25) (layer B.Cu) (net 32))
 (segment (start 163.322 111.76) (end 164.497001 110.584999) (width 0.25) (layer B.Cu) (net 32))
 (segment (start 108.712 101.473) (end 106.426 99.187) (width 0.25) (layer B.Cu) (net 32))
 (segment (start 108.712 102.362) (end 108.712 101.473) (width 0.25) (layer B.Cu) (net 32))
 (segment (start 167.836009 105.604599) (end 167.0644 104.83299) (width 0.25) (layer B.Cu) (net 32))
 (segment (start 167.836009 108.984993) (end 167.836009 105.604599) (width 0.25) (layer B.Cu) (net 32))
 (segment (start 166.426001 110.395001) (end 167.836009 108.984993) (width 0.25) (layer B.Cu) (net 32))
 (segment (start 164.686999 110.395001) (end 166.426001 110.395001) (width 0.25) (layer B.Cu) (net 32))
 (segment (start 163.322 111.76) (end 164.686999 110.395001) (width 0.25) (layer B.Cu) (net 32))
 (segment (start 111.18299 104.83299) (end 110.363 104.013) (width 0.25) (layer B.Cu) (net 32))
 (segment (start 167.0644 104.83299) (end 111.18299 104.83299) (width 0.25) (layer B.Cu) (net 32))
 (segment (start 110.363 104.013) (end 108.712 102.362) (width 0.25) (layer B.Cu) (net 32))
 (segment (start 111.125 104.775) (end 110.363 104.013) (width 0.25) (layer B.Cu) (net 32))
 (segment (start 135.636 76.2) (end 135.636 77.343) (width 0.25) (layer F.Cu) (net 27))
 (segment (start 136.76798 82.53898) (end 135.636 81.407) (width 0.25) (layer F.Cu) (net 27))
 (segment (start 135.636 81.407) (end 135.636 76.2) (width 0.25) (layer F.Cu) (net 27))
 (segment (start 145.27698 82.53898) (end 136.76798 82.53898) (width 0.25) (layer F.Cu) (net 27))
 (segment (start 146.431 83.693) (end 145.27698 82.53898) (width 0.25) (layer F.Cu) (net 27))
 (segment (start 146.431 85.852) (end 146.431 83.693) (width 0.25) (layer F.Cu) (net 27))
 (segment (start 104.350939 89.30097) (end 113.260909 80.391) (width 0.25) (layer B.Cu) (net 27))
 (segment (start 104.350939 101.556939) (end 104.350939 89.30097) (width 0.25) (layer B.Cu) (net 27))
 (segment (start 106.426 103.632) (end 104.350939 101.556939) (width 0.25) (layer B.Cu) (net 27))
 (segment (start 113.260909 80.391) (end 133.35 80.391) (width 0.25) (layer B.Cu) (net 27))
 (segment (start 135.636 78.105) (end 135.636 76.2) (width 0.25) (layer B.Cu) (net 27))
 (segment (start 133.35 80.391) (end 135.636 78.105) (width 0.25) (layer B.Cu) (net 27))
 (segment (start 165.862 109.22) (end 167.386 107.696) (width 0.25) (layer B.Cu) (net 27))
 (segment (start 167.386 107.696) (end 167.386 105.791) (width 0.25) (layer B.Cu) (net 27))
 (segment (start 167.386 105.791) (end 166.878 105.283) (width 0.25) (layer B.Cu) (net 27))
 (segment (start 108.077 105.283) (end 106.426 103.632) (width 0.25) (layer B.Cu) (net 27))
 (segment (start 166.878 105.283) (end 108.077 105.283) (width 0.25) (layer B.Cu) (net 27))
 (segment (start 130.556 82.042) (end 130.556 81.28) (width 0.25) (layer F.Cu) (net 23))
 (segment (start 131.953 83.439) (end 130.556 82.042) (width 0.25) (layer F.Cu) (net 23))
 (segment (start 140.716 83.439) (end 131.953 83.439) (width 0.25) (layer F.Cu) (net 23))
 (segment (start 141.351 84.074) (end 140.716 83.439) (width 0.25) (layer F.Cu) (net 23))
 (segment (start 141.351 85.852) (end 141.351 84.074) (width 0.25) (layer F.Cu) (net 23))
 (segment (start 130.556 81.28) (end 130.556 76.2) (width 0.25) (layer F.Cu) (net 23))
 (segment (start 130.556 81.661) (end 130.556 81.28) (width 0.25) (layer F.Cu) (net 23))
 (segment (start 106.426 112.522) (end 103.45092 109.54692) (width 0.25) (layer B.Cu) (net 23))
 (segment (start 103.45092 109.54692) (end 103.450921 88.928168) (width 0.25) (layer B.Cu) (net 23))
 (segment (start 103.450921 88.928168) (end 112.888109 79.49098) (width 0.25) (layer B.Cu) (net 23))
 (segment (start 112.888109 79.49098) (end 129.17002 79.49098) (width 0.25) (layer B.Cu) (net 23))
 (segment (start 130.556 78.105) (end 130.556 76.2) (width 0.25) (layer B.Cu) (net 23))
 (segment (start 129.17002 79.49098) (end 130.556 78.105) (width 0.25) (layer B.Cu) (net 23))
 (segment (start 109.0295 109.9185) (end 106.426 112.522) (width 0.25) (layer B.Cu) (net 23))
 (segment (start 109.0295 108.1405) (end 109.0295 109.9185) (width 0.25) (layer B.Cu) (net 23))
 (segment (start 110.98698 106.18302) (end 109.0295 108.1405) (width 0.25) (layer B.Cu) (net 23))
 (segment (start 160.28502 106.18302) (end 110.98698 106.18302) (width 0.25) (layer B.Cu) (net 23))
 (segment (start 161.036 108.331) (end 161.036 106.934) (width 0.25) (layer B.Cu) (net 23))
 (segment (start 161.925 109.22) (end 161.036 108.331) (width 0.25) (layer B.Cu) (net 23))
 (segment (start 161.036 106.934) (end 160.28502 106.18302) (width 0.25) (layer B.Cu) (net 23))
 (segment (start 163.322 109.22) (end 161.925 109.22) (width 0.25) (layer B.Cu) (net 23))
 (segment (start 133.096 81.661) (end 133.096 78.359) (width 0.25) (layer F.Cu) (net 25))
 (segment (start 142.93299 82.98899) (end 134.42399 82.98899) (width 0.25) (layer F.Cu) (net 25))
 (segment (start 143.891 83.947) (end 142.93299 82.98899) (width 0.25) (layer F.Cu) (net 25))
 (segment (start 143.891 85.852) (end 143.891 83.947) (width 0.25) (layer F.Cu) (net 25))
 (segment (start 133.096 78.359) (end 133.096 76.2) (width 0.25) (layer F.Cu) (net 25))
 (segment (start 134.42399 82.98899) (end 133.096 81.661) (width 0.25) (layer F.Cu) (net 25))
 (segment (start 133.096 81.026) (end 133.096 78.359) (width 0.25) (layer F.Cu) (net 25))
 (segment (start 106.426 108.077) (end 103.900929 105.551929) (width 0.25) (layer B.Cu) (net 25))
 (segment (start 103.90093 89.114569) (end 113.074509 79.94099) (width 0.25) (layer B.Cu) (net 25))
 (segment (start 103.900929 105.551929) (end 103.90093 89.114569) (width 0.25) (layer B.Cu) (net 25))
 (segment (start 113.074509 79.94099) (end 131.26001 79.94099) (width 0.25) (layer B.Cu) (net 25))
 (segment (start 133.096 78.105) (end 133.096 76.2) (width 0.25) (layer B.Cu) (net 25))
 (segment (start 131.26001 79.94099) (end 133.096 78.105) (width 0.25) (layer B.Cu) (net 25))
 (segment (start 107.7595 106.7435) (end 106.426 108.077) (width 0.25) (layer B.Cu) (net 25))
 (segment (start 162.222 106.68) (end 161.27501 105.73301) (width 0.25) (layer B.Cu) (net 25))
 (segment (start 108.76999 105.73301) (end 107.7595 106.7435) (width 0.25) (layer B.Cu) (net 25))
 (segment (start 161.27501 105.73301) (end 108.76999 105.73301) (width 0.25) (layer B.Cu) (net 25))
 (segment (start 163.322 106.68) (end 162.222 106.68) (width 0.25) (layer B.Cu) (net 25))
 (segment (start 152.4676 78.68201) (end 144.21401 78.68201) (width 0.25) (layer F.Cu) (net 4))
 (segment (start 153.47399 79.6884) (end 152.4676 78.68201) (width 0.25) (layer F.Cu) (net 4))
 (segment (start 154.94 84.07541) (end 153.47399 82.6094) (width 0.25) (layer F.Cu) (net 4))
 (segment (start 154.94 99.695) (end 154.94 84.07541) (width 0.25) (layer F.Cu) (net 4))
 (segment (start 144.21401 78.68201) (end 143.256 77.724) (width 0.25) (layer F.Cu) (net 4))
 (segment (start 155.575 100.33) (end 154.94 99.695) (width 0.25) (layer F.Cu) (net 4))
 (segment (start 143.256 77.724) (end 143.256 76.2) (width 0.25) (layer F.Cu) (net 4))
 (segment (start 153.47399 82.6094) (end 153.47399 79.6884) (width 0.25) (layer F.Cu) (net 4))
 (segment (start 156.6695 100.33) (end 155.575 100.33) (width 0.25) (layer F.Cu) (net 4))
 (segment (start 152.2812 79.13202) (end 141.87002 79.13202) (width 0.25) (layer F.Cu) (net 6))
 (segment (start 153.02398 79.8748) (end 152.2812 79.13202) (width 0.25) (layer F.Cu) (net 6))
 (segment (start 153.02398 82.7958) (end 153.02398 79.8748) (width 0.25) (layer F.Cu) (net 6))
 (segment (start 140.716 77.978) (end 140.716 76.2) (width 0.25) (layer F.Cu) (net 6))
 (segment (start 154.48999 84.26181) (end 153.02398 82.7958) (width 0.25) (layer F.Cu) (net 6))
 (segment (start 154.48999 102.29299) (end 154.48999 84.26181) (width 0.25) (layer F.Cu) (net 6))
 (segment (start 155.067 102.87) (end 154.48999 102.29299) (width 0.25) (layer F.Cu) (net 6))
 (segment (start 141.87002 79.13202) (end 140.716 77.978) (width 0.25) (layer F.Cu) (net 6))
 (segment (start 156.6695 102.87) (end 155.067 102.87) (width 0.25) (layer F.Cu) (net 6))
 (segment (start 156.6695 97.79) (end 156.21 97.79) (width 0.25) (layer F.Cu) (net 2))
 (segment (start 155.89801 97.79) (end 156.6695 97.79) (width 0.25) (layer F.Cu) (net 2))
 (segment (start 155.39001 97.282) (end 155.89801 97.79) (width 0.25) (layer F.Cu) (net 2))
 (segment (start 155.390009 83.889009) (end 155.39001 97.282) (width 0.25) (layer F.Cu) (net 2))
 (segment (start 153.924 82.423) (end 155.390009 83.889009) (width 0.25) (layer F.Cu) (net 2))
 (segment (start 153.924 79.502) (end 153.924 82.423) (width 0.25) (layer F.Cu) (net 2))
 (segment (start 152.654 78.232) (end 153.924 79.502) (width 0.25) (layer F.Cu) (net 2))
 (segment (start 147.32 76.2) (end 147.32 77.47) (width 0.25) (layer F.Cu) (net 2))
 (segment (start 148.082 78.232) (end 152.654 78.232) (width 0.25) (layer F.Cu) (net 2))
 (segment (start 147.32 77.47) (end 148.082 78.232) (width 0.25) (layer F.Cu) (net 2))
 (segment (start 162.3845 102.87) (end 158.5445 102.87) (width 0.25) (layer F.Cu) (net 5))
 (segment (start 162.3845 100.33) (end 158.5445 100.33) (width 0.25) (layer F.Cu) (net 3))
 (segment (start 162.3845 97.79) (end 158.5445 97.79) (width 0.25) (layer F.Cu) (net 1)))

